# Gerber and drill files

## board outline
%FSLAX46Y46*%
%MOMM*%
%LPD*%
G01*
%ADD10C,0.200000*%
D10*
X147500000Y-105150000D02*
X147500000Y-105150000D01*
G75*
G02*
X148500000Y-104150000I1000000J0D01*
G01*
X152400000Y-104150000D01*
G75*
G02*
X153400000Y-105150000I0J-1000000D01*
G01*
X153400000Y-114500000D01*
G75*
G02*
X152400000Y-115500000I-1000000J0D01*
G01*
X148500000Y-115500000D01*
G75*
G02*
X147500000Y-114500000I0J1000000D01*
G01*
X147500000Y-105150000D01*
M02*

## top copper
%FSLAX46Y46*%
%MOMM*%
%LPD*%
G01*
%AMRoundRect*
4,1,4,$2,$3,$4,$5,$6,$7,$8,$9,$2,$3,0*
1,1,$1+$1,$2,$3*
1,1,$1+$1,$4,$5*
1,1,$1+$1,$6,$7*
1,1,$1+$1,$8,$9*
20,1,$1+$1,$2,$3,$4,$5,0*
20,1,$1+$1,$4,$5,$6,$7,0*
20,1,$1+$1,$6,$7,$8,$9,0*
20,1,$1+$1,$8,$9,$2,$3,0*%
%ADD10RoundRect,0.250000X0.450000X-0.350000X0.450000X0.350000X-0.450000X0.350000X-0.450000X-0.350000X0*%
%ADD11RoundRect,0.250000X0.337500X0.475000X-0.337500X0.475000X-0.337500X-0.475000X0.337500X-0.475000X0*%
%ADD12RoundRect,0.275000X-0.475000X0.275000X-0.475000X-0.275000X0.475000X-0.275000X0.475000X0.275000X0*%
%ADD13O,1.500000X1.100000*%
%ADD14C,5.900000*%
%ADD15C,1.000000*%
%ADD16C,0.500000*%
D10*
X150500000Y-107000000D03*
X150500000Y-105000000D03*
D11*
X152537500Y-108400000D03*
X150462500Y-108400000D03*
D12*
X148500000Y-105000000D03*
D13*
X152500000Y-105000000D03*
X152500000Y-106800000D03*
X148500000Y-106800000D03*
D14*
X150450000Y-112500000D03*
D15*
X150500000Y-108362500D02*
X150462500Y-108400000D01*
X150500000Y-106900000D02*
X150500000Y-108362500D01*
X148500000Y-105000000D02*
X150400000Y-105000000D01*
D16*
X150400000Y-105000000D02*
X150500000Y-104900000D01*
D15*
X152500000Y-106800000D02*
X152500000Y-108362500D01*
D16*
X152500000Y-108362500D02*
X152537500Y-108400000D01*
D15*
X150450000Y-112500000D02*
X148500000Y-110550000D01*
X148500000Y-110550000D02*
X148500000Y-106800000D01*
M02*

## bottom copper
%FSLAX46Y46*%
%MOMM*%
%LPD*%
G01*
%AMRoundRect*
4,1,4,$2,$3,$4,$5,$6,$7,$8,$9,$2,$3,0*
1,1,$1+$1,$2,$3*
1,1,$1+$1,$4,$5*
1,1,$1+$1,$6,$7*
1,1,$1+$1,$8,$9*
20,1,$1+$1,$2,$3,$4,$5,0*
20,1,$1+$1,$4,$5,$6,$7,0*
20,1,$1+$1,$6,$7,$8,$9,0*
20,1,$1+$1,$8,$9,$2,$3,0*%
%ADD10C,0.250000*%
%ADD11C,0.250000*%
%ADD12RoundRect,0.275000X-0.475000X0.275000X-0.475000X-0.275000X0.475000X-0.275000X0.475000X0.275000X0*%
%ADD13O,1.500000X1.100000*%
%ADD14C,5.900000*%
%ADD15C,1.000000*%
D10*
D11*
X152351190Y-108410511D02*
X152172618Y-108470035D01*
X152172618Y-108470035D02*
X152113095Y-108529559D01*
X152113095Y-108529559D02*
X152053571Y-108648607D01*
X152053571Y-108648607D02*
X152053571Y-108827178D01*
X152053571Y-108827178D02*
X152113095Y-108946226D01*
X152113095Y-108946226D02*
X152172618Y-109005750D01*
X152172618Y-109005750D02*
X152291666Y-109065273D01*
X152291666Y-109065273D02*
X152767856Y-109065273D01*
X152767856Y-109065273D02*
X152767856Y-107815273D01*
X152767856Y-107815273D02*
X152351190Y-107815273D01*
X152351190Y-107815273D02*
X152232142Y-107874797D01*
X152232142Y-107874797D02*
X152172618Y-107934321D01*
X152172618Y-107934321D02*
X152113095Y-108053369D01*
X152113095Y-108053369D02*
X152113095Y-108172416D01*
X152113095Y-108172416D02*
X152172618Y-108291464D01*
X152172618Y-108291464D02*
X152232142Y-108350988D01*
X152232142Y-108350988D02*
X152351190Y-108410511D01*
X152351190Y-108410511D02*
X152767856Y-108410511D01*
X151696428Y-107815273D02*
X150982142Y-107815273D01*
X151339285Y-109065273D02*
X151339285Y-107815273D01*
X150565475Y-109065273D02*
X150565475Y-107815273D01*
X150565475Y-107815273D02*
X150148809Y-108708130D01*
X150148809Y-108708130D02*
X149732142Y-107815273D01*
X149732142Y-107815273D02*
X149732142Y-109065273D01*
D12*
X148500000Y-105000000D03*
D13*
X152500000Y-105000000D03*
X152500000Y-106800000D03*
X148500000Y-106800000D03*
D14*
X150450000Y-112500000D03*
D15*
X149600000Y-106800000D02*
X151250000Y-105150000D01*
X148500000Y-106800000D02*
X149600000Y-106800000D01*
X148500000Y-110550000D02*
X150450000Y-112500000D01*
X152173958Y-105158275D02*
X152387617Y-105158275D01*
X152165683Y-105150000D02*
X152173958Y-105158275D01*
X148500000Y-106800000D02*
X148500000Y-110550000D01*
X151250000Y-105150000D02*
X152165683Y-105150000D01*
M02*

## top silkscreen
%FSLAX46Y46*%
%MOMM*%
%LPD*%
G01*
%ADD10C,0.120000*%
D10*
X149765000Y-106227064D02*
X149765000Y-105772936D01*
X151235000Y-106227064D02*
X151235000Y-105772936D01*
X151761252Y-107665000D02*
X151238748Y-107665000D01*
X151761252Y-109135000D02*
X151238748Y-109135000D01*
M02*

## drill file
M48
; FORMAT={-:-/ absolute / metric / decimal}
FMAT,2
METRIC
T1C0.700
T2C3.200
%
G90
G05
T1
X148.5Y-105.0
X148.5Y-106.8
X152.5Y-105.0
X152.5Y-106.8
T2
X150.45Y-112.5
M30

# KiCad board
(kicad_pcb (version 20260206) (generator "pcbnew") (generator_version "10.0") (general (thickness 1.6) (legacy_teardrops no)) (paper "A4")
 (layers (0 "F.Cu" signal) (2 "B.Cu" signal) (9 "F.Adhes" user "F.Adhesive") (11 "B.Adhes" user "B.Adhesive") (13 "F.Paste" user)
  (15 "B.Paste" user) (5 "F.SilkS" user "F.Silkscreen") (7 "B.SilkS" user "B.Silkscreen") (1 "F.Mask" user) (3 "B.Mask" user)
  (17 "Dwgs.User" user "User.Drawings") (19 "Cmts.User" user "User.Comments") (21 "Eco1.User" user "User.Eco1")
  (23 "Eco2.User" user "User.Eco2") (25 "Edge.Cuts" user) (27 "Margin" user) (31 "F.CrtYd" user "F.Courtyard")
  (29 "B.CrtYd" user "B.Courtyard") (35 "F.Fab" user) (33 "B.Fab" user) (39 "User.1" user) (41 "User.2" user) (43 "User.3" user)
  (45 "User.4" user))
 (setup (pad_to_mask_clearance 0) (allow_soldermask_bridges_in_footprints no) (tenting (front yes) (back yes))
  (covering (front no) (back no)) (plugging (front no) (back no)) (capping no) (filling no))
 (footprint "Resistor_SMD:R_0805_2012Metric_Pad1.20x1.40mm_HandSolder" (layer "F.Cu") (at 150.5 106 90)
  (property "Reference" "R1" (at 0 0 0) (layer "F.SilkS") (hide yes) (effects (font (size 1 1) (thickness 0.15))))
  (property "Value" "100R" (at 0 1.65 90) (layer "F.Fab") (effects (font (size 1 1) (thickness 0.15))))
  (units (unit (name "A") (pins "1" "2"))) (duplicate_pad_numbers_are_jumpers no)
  (fp_line (start -0.227064 -0.735) (end 0.227064 -0.735) (stroke (width 0.12) (type solid)) (layer "F.SilkS"))
  (fp_line (start -0.227064 0.735) (end 0.227064 0.735) (stroke (width 0.12) (type solid)) (layer "F.SilkS"))
  (pad "1" smd roundrect (at -1 0 90) (size 1.2 1.4) (layers "F.Cu" "F.Mask" "F.Paste") (roundrect_rratio 0.208333) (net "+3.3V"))
  (pad "2" smd roundrect (at 1 0 90) (size 1.2 1.4) (layers "F.Cu" "F.Mask" "F.Paste") (roundrect_rratio 0.208333) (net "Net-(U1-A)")))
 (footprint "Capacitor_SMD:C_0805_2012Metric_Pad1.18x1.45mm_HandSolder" (layer "F.Cu") (at 151.5 108.4 180)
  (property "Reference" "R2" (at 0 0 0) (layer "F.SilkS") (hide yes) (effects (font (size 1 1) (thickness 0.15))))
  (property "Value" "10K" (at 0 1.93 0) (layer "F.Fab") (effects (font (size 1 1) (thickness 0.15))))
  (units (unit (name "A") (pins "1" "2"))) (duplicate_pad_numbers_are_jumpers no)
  (fp_line (start -0.261252 0.735) (end 0.261252 0.735) (stroke (width 0.12) (type solid)) (layer "F.SilkS"))
  (fp_line (start -0.261252 -0.735) (end 0.261252 -0.735) (stroke (width 0.12) (type solid)) (layer "F.SilkS"))
  (pad "1" smd roundrect (at -1.0375 0 180) (size 1.175 1.45) (layers "F.Cu" "F.Mask" "F.Paste") (roundrect_rratio 0.212766)
   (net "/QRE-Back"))
  (pad "2" smd roundrect (at 1.0375 0 180) (size 1.175 1.45) (layers "F.Cu" "F.Mask" "F.Paste") (roundrect_rratio 0.212766) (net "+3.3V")))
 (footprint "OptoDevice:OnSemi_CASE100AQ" (layer "B.Cu") (at 148.5 105 -90)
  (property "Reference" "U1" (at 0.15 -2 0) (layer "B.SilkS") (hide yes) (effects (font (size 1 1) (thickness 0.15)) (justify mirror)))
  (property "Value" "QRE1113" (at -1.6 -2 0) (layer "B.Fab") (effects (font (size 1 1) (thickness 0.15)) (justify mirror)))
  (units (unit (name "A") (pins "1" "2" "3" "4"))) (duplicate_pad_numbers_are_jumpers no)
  (pad "1" thru_hole roundrect (at 0 0 270) (size 1.1 1.5) (drill 0.7) (layers "*.Cu" "*.Mask") (remove_unused_layers no)
   (roundrect_rratio 0.25) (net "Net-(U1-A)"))
  (pad "2" thru_hole oval (at 0 -4 270) (size 1.1 1.5) (drill 0.7) (layers "*.Cu" "*.Mask") (remove_unused_layers no) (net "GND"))
  (pad "3" thru_hole oval (at 1.8 -4 270) (size 1.1 1.5) (drill 0.7) (layers "*.Cu" "*.Mask") (remove_unused_layers no) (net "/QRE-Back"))
  (pad "4" thru_hole oval (at 1.8 0 270) (size 1.1 1.5) (drill 0.7) (layers "*.Cu" "*.Mask") (remove_unused_layers no) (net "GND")))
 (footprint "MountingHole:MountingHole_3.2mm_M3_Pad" (layer "B.Cu") (at 150.45 112.5 180)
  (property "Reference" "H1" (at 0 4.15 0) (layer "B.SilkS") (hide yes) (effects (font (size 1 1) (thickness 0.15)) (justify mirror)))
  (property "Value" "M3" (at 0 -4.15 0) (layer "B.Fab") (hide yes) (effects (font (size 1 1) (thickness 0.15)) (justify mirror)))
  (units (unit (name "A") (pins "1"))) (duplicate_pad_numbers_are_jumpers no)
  (pad "1" thru_hole circle (at 0 0 180) (size 5.9 5.9) (drill 3.2) (layers "*.Cu" "*.Mask") (remove_unused_layers no) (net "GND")
   (zone_connect 2)))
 (gr_rect (start 147.5 104.15) (end 153.4 115.5) (radius 1) (stroke (width 0.2) (type solid)) (fill no) (layer "Edge.Cuts"))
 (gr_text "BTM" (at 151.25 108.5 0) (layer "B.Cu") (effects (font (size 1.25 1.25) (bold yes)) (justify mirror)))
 (segment (start 150.5 108.3625) (end 150.4625 108.4) (width 1) (layer "F.Cu") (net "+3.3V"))
 (segment (start 150.5 106.9) (end 150.5 108.3625) (width 1) (layer "F.Cu") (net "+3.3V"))
 (segment (start 148.5 105) (end 150.4 105) (width 1) (layer "F.Cu") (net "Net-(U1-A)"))
 (segment (start 150.4 105) (end 150.5 104.9) (width 0.5) (layer "F.Cu") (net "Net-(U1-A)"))
 (segment (start 152.5 106.8) (end 152.5 108.3625) (width 1) (layer "F.Cu") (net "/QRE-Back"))
 (segment (start 152.5 108.3625) (end 152.5375 108.4) (width 0.5) (layer "F.Cu") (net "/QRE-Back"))
 (segment (start 150.45 112.5) (end 148.5 110.55) (width 1) (layer "F.Cu") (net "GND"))
 (segment (start 148.5 110.55) (end 148.5 106.8) (width 1) (layer "F.Cu") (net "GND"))
 (segment (start 149.6 106.8) (end 151.25 105.15) (width 1) (layer "B.Cu") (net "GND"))
 (segment (start 148.5 106.8) (end 149.6 106.8) (width 1) (layer "B.Cu") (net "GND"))
 (segment (start 148.5 110.55) (end 150.45 112.5) (width 1) (layer "B.Cu") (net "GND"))
 (segment (start 152.173958 105.158275) (end 152.387617 105.158275) (width 1) (layer "B.Cu") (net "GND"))
 (segment (start 152.165683 105.15) (end 152.173958 105.158275) (width 1) (layer "B.Cu") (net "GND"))
 (segment (start 148.5 106.8) (end 148.5 110.55) (width 1) (layer "B.Cu") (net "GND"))
 (segment (start 151.25 105.15) (end 152.165683 105.15) (width 1) (layer "B.Cu") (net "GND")))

